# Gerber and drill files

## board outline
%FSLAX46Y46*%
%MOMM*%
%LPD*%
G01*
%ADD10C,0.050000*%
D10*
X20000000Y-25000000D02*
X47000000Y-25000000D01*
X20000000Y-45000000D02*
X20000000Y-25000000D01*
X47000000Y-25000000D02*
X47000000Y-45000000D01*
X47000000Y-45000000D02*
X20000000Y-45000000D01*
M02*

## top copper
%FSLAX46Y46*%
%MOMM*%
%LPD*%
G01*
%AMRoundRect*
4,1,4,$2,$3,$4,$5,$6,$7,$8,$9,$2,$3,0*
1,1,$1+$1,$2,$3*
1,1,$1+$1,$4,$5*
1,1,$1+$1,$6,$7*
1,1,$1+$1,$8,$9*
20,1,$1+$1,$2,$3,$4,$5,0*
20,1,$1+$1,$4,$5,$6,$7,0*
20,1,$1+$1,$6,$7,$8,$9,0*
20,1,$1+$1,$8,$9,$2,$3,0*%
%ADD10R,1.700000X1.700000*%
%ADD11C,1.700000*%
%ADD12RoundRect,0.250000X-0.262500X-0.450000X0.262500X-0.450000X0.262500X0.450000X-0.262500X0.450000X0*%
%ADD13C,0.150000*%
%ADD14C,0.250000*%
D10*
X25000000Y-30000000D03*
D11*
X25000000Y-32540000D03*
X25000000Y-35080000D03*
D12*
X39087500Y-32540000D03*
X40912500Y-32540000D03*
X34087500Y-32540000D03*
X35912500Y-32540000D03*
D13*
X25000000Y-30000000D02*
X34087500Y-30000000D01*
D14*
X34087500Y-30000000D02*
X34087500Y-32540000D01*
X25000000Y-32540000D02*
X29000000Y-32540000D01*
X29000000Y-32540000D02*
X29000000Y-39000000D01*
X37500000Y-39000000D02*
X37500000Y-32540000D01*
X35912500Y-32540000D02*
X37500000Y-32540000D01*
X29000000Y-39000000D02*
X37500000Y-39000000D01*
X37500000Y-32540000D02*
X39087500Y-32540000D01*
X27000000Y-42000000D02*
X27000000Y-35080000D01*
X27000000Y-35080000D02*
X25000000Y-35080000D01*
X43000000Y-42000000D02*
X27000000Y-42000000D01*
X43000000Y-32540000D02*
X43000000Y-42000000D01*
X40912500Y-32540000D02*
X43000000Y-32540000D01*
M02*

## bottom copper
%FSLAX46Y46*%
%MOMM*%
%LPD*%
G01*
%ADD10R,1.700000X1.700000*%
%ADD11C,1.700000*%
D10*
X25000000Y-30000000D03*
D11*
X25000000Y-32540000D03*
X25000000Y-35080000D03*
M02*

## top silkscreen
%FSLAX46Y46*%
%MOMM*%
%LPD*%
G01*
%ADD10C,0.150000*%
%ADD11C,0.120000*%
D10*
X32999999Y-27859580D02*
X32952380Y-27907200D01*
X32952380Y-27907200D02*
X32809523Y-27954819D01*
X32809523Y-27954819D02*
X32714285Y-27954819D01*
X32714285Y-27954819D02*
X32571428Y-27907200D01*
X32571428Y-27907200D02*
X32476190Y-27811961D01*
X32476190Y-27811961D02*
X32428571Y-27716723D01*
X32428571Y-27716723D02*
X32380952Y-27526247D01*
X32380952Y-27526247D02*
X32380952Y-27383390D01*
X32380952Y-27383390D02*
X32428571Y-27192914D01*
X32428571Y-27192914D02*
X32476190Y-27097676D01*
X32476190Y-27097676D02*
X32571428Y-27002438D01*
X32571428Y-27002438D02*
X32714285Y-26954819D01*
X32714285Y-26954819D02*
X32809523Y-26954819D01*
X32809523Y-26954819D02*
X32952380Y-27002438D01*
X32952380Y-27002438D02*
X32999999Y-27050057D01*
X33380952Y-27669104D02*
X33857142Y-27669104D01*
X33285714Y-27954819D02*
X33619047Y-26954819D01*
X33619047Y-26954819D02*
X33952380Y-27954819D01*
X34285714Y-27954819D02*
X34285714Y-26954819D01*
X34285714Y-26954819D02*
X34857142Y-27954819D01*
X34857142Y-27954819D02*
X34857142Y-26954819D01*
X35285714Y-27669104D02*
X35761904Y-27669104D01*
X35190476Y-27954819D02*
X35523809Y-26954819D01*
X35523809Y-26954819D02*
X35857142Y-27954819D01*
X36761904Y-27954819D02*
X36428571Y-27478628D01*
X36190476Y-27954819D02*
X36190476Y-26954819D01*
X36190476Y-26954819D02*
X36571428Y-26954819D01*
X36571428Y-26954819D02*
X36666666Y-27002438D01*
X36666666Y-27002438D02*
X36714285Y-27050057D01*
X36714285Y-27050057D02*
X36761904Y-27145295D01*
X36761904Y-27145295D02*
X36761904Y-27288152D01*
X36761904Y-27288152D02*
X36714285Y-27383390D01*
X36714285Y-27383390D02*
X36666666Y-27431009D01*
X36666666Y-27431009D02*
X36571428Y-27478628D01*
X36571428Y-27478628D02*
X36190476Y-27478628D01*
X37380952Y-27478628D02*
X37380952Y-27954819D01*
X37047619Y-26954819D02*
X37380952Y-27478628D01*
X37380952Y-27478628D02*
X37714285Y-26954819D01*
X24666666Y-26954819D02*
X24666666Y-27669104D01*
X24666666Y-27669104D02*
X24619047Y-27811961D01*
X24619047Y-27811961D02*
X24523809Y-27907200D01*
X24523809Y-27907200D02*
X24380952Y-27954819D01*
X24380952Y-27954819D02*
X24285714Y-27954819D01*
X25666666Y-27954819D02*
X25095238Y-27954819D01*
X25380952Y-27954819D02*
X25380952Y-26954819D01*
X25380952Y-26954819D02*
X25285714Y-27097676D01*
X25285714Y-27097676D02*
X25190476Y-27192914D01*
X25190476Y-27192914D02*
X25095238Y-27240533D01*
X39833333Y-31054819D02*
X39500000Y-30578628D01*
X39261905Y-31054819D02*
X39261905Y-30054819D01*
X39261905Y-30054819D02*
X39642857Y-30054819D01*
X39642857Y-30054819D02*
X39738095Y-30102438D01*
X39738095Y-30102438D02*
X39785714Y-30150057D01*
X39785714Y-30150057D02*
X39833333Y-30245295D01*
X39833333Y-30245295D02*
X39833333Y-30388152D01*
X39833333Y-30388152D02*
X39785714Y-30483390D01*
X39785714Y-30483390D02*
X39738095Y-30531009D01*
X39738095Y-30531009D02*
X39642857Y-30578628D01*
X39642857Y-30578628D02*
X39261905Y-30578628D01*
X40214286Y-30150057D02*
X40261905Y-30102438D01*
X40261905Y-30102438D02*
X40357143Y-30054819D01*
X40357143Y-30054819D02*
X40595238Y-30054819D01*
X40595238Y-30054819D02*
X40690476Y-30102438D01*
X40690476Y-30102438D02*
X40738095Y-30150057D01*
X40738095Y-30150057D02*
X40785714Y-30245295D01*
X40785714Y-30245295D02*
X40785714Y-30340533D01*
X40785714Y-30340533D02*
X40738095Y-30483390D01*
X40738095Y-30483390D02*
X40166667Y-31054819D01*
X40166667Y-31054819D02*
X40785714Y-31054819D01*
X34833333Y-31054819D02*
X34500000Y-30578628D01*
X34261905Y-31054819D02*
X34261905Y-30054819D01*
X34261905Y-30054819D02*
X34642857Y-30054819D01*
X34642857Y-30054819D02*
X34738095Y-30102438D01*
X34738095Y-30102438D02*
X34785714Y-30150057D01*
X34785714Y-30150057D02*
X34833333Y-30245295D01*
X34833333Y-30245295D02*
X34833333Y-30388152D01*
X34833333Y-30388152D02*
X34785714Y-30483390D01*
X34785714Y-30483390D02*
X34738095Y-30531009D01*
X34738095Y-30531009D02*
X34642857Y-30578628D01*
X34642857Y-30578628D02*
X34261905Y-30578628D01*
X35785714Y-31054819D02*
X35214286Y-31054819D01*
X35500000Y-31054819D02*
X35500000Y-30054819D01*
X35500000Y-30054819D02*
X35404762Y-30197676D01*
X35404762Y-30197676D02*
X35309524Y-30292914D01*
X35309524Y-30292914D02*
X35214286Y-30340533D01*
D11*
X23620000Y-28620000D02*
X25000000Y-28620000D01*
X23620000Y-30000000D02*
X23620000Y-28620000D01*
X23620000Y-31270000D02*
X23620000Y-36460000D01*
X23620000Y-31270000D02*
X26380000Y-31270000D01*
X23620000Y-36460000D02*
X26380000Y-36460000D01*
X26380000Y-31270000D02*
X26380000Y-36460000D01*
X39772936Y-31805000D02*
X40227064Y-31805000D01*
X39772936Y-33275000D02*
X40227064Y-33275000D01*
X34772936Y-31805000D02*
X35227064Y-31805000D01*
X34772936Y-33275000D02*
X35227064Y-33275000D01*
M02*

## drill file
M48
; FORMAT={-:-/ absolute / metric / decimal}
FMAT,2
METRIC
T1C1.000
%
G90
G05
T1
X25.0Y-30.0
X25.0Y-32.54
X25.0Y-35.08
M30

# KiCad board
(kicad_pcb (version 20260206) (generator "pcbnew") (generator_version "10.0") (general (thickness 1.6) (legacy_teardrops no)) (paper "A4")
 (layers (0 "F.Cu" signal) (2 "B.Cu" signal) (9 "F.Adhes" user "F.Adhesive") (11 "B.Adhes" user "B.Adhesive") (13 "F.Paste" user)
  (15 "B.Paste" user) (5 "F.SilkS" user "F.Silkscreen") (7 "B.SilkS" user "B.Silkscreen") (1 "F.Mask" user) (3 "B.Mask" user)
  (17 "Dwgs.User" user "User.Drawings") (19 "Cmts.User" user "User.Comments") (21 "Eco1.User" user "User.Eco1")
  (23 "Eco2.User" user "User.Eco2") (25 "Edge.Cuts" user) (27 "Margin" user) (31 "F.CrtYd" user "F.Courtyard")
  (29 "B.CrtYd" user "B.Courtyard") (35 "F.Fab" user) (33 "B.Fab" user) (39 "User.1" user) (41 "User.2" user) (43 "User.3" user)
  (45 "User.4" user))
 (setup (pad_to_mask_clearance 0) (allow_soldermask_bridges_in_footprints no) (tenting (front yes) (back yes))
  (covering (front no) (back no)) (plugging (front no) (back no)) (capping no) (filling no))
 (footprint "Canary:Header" (layer "F.Cu") (at 25 30)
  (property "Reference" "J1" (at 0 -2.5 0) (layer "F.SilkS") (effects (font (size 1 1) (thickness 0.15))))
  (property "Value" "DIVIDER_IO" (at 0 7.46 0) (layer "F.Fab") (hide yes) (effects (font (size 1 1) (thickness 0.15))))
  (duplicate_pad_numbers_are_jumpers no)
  (fp_line (start -1.38 -1.38) (end 0 -1.38) (stroke (width 0.12) (type solid)) (layer "F.SilkS"))
  (fp_line (start -1.38 0) (end -1.38 -1.38) (stroke (width 0.12) (type solid)) (layer "F.SilkS"))
  (fp_line (start -1.38 1.27) (end -1.38 6.46) (stroke (width 0.12) (type solid)) (layer "F.SilkS"))
  (fp_line (start -1.38 1.27) (end 1.38 1.27) (stroke (width 0.12) (type solid)) (layer "F.SilkS"))
  (fp_line (start -1.38 6.46) (end 1.38 6.46) (stroke (width 0.12) (type solid)) (layer "F.SilkS"))
  (fp_line (start 1.38 1.27) (end 1.38 6.46) (stroke (width 0.12) (type solid)) (layer "F.SilkS"))
  (pad "1" thru_hole rect (at 0 0) (size 1.7 1.7) (drill 1) (layers "*.Cu" "*.Mask") (remove_unused_layers no) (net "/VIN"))
  (pad "2" thru_hole circle (at 0 2.54) (size 1.7 1.7) (drill 1) (layers "*.Cu" "*.Mask") (remove_unused_layers no) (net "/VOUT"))
  (pad "3" thru_hole circle (at 0 5.08) (size 1.7 1.7) (drill 1) (layers "*.Cu" "*.Mask") (remove_unused_layers no) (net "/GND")))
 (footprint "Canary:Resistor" (layer "F.Cu") (at 40 32.54)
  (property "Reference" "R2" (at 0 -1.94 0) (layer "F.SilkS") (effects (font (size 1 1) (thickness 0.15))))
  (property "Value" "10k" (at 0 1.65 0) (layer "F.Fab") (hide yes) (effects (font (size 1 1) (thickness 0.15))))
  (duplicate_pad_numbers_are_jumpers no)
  (fp_line (start -0.227064 -0.735) (end 0.227064 -0.735) (stroke (width 0.12) (type solid)) (layer "F.SilkS"))
  (fp_line (start -0.227064 0.735) (end 0.227064 0.735) (stroke (width 0.12) (type solid)) (layer "F.SilkS"))
  (pad "1" smd roundrect (at -0.9125 0) (size 1.025 1.4) (layers "F.Cu" "F.Mask" "F.Paste") (roundrect_rratio 0.243902) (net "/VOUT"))
  (pad "2" smd roundrect (at 0.9125 0) (size 1.025 1.4) (layers "F.Cu" "F.Mask" "F.Paste") (roundrect_rratio 0.243902) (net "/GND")))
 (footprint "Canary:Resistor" (layer "F.Cu") (at 35 32.54)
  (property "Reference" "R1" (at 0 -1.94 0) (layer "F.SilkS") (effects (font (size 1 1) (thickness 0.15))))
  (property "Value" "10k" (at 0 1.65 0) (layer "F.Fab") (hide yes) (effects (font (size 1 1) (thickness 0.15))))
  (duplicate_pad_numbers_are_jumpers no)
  (fp_line (start -0.227064 -0.735) (end 0.227064 -0.735) (stroke (width 0.12) (type solid)) (layer "F.SilkS"))
  (fp_line (start -0.227064 0.735) (end 0.227064 0.735) (stroke (width 0.12) (type solid)) (layer "F.SilkS"))
  (pad "1" smd roundrect (at -0.9125 0) (size 1.025 1.4) (layers "F.Cu" "F.Mask" "F.Paste") (roundrect_rratio 0.243902) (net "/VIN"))
  (pad "2" smd roundrect (at 0.9125 0) (size 1.025 1.4) (layers "F.Cu" "F.Mask" "F.Paste") (roundrect_rratio 0.243902) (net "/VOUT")))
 (gr_line (start 20 25) (end 47 25) (stroke (width 0.05) (type default)) (layer "Edge.Cuts"))
 (gr_line (start 20 45) (end 20 25) (stroke (width 0.05) (type default)) (layer "Edge.Cuts"))
 (gr_line (start 47 25) (end 47 45) (stroke (width 0.05) (type default)) (layer "Edge.Cuts"))
 (gr_line (start 47 45) (end 20 45) (stroke (width 0.05) (type default)) (layer "Edge.Cuts"))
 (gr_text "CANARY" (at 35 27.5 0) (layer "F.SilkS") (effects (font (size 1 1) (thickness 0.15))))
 (segment (start 25 30) (end 34.0875 30) (width 0.15) (layer "F.Cu") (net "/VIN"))
 (segment (start 34.0875 30) (end 34.0875 32.54) (width 0.25) (layer "F.Cu") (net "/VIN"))
 (segment (start 25 32.54) (end 29 32.54) (width 0.25) (layer "F.Cu") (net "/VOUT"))
 (segment (start 29 32.54) (end 29 39) (width 0.25) (layer "F.Cu") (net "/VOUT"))
 (segment (start 37.5 39) (end 37.5 32.54) (width 0.25) (layer "F.Cu") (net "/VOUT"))
 (segment (start 35.9125 32.54) (end 37.5 32.54) (width 0.25) (layer "F.Cu") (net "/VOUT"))
 (segment (start 29 39) (end 37.5 39) (width 0.25) (layer "F.Cu") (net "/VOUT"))
 (segment (start 37.5 32.54) (end 39.0875 32.54) (width 0.25) (layer "F.Cu") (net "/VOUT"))
 (segment (start 27 42) (end 27 35.08) (width 0.25) (layer "F.Cu") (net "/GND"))
 (segment (start 27 35.08) (end 25 35.08) (width 0.25) (layer "F.Cu") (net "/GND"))
 (segment (start 43 42) (end 27 42) (width 0.25) (layer "F.Cu") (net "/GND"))
 (segment (start 43 32.54) (end 43 42) (width 0.25) (layer "F.Cu") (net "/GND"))
 (segment (start 40.9125 32.54) (end 43 32.54) (width 0.25) (layer "F.Cu") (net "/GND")))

